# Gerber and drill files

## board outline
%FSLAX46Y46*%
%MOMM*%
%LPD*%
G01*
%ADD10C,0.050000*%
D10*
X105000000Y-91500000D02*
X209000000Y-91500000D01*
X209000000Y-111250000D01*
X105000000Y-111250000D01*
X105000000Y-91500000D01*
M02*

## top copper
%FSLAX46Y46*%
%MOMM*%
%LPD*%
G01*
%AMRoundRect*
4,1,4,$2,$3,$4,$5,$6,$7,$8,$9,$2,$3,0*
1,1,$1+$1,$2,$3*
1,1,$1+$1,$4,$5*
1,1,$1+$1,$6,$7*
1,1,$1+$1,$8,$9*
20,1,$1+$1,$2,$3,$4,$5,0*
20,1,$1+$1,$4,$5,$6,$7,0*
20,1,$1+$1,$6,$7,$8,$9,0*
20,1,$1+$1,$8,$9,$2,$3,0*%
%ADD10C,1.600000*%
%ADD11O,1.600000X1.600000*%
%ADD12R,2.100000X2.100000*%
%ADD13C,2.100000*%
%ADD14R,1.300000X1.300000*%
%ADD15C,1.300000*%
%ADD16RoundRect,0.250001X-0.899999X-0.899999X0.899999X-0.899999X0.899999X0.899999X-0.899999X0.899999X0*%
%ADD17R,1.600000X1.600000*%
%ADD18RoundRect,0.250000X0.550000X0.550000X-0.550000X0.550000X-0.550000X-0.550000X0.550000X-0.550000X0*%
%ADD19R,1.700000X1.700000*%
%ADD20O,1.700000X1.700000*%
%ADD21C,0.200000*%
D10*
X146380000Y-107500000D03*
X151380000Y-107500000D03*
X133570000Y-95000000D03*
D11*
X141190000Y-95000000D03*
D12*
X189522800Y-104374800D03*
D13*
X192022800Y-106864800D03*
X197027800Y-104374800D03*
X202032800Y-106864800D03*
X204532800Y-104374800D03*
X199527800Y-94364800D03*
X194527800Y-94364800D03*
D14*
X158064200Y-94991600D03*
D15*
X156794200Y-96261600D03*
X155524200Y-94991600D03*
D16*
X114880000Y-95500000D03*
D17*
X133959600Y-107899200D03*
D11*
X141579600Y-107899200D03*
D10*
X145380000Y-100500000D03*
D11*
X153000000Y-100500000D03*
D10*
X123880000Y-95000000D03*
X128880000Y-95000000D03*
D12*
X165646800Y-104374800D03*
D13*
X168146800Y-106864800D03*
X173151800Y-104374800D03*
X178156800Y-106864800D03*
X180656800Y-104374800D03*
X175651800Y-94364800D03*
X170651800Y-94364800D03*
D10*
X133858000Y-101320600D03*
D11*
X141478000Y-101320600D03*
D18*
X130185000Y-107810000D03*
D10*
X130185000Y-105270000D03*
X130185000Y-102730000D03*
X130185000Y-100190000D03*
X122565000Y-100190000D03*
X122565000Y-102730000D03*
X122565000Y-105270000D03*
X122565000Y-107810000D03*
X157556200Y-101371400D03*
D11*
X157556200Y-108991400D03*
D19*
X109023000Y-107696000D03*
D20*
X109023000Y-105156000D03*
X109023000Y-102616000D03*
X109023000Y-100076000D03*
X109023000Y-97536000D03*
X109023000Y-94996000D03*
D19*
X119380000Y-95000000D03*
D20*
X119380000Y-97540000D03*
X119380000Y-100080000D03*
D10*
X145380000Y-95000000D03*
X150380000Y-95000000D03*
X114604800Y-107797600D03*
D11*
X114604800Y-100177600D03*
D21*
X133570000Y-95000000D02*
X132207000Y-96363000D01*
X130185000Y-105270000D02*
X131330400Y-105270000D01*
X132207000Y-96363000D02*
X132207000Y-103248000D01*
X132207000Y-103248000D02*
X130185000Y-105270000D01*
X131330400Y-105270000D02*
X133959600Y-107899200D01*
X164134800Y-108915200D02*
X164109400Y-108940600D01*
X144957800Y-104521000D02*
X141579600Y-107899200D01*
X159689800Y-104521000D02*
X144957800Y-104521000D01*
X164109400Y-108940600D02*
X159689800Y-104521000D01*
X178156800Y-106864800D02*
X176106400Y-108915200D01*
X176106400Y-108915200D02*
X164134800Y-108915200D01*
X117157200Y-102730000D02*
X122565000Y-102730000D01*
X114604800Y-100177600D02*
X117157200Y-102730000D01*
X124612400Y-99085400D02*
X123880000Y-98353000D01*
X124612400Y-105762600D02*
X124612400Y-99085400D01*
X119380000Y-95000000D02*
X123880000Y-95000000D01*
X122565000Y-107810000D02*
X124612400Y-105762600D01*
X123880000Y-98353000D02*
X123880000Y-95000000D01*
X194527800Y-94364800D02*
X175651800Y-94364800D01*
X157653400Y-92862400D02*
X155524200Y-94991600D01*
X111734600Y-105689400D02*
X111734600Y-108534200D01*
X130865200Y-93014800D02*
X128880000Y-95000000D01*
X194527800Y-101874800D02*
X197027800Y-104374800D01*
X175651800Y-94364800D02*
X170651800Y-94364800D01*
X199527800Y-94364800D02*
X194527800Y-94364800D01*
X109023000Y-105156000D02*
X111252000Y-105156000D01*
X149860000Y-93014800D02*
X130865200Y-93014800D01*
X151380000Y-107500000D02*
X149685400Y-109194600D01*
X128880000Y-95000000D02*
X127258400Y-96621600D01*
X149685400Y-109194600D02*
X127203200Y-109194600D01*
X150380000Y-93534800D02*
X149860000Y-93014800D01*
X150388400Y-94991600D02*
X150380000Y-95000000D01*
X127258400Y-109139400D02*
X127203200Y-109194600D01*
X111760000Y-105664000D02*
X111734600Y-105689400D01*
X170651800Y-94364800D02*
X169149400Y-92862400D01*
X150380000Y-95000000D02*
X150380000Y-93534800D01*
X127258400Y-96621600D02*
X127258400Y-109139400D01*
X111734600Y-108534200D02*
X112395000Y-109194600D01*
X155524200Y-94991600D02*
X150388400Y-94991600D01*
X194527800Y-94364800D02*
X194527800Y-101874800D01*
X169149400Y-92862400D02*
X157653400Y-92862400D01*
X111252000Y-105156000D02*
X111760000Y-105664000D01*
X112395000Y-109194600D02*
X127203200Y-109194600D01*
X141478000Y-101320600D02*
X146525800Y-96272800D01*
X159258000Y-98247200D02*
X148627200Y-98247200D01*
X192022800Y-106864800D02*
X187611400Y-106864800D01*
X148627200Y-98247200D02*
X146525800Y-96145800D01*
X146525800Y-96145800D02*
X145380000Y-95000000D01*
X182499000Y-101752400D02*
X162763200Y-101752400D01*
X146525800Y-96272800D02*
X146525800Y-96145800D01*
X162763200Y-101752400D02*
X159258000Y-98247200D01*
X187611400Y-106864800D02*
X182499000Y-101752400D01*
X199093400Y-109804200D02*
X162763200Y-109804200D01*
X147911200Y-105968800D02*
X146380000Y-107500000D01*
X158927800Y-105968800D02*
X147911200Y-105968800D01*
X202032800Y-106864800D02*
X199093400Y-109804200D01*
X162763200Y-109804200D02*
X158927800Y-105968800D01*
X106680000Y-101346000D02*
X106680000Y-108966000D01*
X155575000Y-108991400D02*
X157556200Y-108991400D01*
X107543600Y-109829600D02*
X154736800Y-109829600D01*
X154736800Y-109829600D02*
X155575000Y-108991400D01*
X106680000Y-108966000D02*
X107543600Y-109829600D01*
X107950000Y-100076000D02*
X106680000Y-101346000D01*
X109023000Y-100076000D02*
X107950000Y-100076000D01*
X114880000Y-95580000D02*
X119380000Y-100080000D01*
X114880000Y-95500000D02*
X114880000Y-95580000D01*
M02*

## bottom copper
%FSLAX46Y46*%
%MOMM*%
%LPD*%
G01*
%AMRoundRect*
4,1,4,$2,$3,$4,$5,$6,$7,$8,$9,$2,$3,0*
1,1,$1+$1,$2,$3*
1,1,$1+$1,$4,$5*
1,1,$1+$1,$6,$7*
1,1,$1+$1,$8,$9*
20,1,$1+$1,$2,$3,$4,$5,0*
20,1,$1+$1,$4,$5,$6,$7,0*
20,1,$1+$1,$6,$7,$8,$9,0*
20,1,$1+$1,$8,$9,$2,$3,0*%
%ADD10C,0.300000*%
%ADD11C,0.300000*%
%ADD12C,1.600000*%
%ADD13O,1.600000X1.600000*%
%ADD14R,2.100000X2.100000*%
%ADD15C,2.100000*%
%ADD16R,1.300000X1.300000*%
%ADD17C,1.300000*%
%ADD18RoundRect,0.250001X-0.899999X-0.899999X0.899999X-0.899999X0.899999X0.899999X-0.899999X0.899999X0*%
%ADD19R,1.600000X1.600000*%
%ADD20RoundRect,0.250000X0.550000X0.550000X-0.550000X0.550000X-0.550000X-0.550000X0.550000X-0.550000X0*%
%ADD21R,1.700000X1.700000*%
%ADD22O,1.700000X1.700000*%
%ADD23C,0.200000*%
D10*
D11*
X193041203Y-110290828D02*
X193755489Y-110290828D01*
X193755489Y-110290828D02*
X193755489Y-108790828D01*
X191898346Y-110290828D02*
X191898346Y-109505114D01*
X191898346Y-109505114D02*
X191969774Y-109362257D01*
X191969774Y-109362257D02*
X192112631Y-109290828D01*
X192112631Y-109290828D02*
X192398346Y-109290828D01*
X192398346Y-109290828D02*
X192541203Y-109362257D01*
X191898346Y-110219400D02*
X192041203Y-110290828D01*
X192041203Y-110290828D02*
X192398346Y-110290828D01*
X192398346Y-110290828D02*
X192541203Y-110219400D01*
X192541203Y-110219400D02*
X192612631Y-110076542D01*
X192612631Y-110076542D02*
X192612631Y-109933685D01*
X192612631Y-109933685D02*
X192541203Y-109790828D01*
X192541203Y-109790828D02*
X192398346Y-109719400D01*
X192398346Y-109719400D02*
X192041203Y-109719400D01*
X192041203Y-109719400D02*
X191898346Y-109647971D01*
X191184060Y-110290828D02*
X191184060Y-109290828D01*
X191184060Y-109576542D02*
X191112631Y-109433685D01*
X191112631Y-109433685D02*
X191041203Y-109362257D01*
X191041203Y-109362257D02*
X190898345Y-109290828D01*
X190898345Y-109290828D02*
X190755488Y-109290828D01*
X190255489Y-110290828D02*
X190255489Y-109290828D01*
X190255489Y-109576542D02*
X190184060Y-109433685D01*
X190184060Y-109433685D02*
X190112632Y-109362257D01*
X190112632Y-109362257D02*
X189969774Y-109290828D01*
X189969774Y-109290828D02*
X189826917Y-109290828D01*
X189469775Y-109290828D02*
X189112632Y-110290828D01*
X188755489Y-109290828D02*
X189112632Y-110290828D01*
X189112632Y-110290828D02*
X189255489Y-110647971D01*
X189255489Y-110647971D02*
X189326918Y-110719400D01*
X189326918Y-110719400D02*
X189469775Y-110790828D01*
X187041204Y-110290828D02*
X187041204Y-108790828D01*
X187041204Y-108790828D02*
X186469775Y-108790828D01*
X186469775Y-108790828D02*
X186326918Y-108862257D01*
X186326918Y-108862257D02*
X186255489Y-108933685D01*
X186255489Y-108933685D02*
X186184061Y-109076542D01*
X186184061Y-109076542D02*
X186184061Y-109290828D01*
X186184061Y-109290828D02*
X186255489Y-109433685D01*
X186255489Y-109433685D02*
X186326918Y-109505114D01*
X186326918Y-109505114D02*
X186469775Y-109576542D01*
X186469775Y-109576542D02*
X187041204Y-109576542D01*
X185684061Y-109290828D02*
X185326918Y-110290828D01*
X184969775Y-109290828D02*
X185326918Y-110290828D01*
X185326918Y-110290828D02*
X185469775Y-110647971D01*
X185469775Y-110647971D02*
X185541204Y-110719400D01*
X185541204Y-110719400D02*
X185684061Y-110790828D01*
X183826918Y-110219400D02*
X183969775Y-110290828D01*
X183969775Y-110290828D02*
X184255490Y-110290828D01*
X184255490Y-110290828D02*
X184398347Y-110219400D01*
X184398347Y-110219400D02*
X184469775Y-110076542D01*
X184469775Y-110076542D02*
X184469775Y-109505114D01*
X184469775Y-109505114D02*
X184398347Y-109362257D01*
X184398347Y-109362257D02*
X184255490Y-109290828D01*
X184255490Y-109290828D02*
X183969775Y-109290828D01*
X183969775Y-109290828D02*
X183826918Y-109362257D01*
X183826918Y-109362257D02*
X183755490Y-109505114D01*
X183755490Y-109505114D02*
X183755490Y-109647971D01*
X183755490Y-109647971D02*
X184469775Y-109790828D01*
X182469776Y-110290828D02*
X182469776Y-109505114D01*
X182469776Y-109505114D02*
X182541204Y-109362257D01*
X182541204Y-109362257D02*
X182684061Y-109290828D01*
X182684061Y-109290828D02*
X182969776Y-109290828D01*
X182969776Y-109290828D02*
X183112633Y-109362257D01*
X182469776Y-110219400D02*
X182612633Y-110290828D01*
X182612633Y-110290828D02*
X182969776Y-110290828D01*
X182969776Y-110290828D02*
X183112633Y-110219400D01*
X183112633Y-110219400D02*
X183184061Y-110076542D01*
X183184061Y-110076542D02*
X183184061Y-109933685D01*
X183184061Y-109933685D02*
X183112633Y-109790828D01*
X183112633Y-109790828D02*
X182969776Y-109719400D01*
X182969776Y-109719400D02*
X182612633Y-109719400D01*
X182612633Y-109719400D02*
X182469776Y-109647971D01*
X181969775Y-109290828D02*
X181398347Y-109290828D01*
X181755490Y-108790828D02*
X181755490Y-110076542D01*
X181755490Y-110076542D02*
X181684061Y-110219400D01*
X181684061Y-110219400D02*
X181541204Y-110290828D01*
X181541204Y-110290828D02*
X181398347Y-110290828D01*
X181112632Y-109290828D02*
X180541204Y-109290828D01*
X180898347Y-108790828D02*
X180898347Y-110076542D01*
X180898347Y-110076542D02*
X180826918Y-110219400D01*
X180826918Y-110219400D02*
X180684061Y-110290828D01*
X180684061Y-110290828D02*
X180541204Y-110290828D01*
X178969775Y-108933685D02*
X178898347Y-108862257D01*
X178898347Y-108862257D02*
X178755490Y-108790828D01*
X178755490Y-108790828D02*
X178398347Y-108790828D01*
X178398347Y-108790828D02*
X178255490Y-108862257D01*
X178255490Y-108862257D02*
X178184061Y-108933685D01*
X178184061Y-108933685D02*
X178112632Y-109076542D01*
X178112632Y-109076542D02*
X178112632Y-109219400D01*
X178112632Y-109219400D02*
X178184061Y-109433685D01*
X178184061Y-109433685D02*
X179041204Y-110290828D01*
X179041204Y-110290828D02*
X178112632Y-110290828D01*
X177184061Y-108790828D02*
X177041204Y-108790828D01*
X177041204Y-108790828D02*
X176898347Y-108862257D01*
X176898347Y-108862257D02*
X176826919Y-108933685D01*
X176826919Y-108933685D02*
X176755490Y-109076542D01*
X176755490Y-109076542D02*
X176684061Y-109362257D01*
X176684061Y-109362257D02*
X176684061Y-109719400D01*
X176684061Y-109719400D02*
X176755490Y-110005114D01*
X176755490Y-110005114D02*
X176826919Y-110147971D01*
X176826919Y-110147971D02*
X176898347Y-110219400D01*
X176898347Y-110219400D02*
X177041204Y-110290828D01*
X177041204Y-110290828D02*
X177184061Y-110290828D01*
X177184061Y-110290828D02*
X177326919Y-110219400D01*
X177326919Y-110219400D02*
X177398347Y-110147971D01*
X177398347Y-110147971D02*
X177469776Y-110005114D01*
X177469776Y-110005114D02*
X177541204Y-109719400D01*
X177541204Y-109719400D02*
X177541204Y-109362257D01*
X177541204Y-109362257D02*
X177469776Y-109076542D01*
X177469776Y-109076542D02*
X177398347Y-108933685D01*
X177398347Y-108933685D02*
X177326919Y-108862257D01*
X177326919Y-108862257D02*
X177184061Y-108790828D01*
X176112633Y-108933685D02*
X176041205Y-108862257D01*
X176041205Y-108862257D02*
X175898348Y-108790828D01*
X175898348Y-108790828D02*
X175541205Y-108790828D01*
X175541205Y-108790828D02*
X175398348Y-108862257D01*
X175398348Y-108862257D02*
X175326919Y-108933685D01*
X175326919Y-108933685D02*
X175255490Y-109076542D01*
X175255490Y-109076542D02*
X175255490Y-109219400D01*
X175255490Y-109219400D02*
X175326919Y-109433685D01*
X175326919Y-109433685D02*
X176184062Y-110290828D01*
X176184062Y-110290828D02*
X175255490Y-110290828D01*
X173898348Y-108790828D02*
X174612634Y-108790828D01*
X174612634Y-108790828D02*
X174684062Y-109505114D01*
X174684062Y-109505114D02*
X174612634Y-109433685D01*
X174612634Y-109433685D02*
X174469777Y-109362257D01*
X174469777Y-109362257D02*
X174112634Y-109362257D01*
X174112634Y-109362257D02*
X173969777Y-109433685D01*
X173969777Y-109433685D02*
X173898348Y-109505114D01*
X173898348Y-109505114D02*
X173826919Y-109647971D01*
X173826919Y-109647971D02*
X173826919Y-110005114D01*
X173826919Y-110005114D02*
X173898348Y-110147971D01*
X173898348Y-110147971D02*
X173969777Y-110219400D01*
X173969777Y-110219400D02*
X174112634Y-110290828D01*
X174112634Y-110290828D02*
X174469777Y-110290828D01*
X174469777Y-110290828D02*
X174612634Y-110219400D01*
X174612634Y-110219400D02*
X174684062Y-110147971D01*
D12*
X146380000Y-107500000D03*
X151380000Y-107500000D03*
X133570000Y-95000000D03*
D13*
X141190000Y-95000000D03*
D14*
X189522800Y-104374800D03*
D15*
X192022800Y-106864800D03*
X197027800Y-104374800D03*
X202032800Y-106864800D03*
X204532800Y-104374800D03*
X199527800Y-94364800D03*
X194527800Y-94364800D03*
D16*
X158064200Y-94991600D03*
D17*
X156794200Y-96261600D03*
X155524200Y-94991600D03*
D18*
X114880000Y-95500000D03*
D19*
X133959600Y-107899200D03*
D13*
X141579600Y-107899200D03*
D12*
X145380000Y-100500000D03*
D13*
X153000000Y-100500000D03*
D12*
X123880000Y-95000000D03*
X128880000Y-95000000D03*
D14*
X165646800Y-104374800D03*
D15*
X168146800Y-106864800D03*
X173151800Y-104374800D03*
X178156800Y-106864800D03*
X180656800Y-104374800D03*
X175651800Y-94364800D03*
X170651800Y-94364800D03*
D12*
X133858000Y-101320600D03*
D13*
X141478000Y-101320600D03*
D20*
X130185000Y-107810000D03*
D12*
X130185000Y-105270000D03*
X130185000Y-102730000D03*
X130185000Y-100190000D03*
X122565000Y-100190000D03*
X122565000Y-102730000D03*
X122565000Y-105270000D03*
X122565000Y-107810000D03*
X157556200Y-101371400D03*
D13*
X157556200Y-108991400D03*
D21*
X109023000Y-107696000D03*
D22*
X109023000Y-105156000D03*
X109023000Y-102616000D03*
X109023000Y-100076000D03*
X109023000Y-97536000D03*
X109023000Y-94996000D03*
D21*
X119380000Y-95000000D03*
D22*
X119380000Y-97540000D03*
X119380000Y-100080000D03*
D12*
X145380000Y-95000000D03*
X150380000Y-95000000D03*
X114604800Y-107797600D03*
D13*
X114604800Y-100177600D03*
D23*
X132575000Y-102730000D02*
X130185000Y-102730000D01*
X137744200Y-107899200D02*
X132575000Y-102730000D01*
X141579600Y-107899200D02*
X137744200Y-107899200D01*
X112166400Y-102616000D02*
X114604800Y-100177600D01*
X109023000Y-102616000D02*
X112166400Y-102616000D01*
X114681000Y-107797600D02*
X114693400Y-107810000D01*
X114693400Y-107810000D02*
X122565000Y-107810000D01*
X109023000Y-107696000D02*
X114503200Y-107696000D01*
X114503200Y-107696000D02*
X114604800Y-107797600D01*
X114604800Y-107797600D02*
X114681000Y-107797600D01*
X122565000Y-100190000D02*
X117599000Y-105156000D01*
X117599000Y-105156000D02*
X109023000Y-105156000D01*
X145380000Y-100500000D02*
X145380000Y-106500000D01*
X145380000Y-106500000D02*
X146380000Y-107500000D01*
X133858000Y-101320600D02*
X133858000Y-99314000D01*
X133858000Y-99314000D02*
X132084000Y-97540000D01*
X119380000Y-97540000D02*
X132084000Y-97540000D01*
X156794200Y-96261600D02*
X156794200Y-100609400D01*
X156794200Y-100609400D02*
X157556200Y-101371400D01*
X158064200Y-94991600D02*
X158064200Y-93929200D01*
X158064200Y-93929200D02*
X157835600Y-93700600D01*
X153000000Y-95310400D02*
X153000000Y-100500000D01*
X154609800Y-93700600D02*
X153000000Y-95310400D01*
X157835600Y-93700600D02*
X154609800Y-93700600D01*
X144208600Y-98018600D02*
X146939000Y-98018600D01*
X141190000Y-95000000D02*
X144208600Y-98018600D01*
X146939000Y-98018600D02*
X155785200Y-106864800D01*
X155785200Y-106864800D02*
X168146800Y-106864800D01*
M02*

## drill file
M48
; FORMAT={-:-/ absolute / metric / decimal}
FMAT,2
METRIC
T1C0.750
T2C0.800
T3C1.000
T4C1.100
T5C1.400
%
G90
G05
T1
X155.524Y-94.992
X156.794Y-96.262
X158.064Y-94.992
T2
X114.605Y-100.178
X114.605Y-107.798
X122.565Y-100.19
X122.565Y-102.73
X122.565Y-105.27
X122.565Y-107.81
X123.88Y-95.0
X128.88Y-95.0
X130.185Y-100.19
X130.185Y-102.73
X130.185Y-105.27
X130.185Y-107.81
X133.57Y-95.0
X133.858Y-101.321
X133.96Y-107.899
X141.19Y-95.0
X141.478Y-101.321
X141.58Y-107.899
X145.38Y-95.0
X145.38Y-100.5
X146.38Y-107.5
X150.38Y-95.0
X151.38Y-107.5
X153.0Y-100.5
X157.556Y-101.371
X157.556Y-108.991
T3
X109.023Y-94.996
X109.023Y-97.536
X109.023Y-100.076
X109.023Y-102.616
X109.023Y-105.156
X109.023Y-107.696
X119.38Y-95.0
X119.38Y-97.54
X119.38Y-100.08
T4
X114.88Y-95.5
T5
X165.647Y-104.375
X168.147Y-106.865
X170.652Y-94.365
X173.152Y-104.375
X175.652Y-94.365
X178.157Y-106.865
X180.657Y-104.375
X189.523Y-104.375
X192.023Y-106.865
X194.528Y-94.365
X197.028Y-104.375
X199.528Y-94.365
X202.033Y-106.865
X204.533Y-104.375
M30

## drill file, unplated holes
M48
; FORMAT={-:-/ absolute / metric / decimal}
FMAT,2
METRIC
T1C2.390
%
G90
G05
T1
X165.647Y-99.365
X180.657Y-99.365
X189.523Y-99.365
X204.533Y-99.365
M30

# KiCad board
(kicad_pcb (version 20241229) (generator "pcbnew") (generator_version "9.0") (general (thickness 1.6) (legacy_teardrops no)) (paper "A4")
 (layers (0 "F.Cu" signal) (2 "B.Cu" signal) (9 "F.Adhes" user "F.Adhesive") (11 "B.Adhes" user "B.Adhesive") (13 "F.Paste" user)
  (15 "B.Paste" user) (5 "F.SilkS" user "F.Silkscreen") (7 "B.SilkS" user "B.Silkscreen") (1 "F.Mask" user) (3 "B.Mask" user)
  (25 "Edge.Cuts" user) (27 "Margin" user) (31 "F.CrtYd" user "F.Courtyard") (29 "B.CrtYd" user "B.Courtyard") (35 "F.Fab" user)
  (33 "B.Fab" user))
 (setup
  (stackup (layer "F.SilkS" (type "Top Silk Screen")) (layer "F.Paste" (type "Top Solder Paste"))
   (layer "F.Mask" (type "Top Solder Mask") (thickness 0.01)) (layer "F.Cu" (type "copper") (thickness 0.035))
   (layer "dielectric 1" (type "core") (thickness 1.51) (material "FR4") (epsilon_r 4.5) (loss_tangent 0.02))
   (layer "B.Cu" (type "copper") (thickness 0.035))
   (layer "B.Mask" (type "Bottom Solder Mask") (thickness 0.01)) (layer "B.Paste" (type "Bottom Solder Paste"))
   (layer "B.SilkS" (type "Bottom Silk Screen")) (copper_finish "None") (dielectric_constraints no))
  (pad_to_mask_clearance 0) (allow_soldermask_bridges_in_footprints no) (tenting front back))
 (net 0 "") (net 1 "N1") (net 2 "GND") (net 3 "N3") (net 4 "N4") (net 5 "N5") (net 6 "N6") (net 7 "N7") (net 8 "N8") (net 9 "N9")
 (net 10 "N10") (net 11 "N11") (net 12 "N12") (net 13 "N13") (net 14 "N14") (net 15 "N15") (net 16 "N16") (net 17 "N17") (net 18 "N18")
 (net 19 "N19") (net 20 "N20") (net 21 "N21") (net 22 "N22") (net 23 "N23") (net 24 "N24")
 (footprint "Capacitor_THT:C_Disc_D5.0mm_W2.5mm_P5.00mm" (layer "F.Cu") (at 146.38 107.5)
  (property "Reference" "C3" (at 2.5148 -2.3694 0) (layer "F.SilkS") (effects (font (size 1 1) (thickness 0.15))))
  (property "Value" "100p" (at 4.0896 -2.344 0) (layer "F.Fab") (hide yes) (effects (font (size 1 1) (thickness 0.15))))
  (pad "1" thru_hole circle (at 0 0) (size 1.6 1.6) (drill 0.8) (layers "*.Cu" "*.Mask") (remove_unused_layers no) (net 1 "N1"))
  (pad "2" thru_hole circle (at 5 0) (size 1.6 1.6) (drill 0.8) (layers "*.Cu" "*.Mask") (remove_unused_layers no) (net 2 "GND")))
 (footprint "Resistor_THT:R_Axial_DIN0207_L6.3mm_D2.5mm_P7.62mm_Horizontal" (layer "F.Cu") (at 133.57 95)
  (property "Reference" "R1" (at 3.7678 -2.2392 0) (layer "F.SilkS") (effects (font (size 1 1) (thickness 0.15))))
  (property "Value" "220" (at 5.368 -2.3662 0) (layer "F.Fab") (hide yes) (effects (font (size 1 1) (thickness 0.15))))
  (pad "1" thru_hole circle (at 0 0) (size 1.6 1.6) (drill 0.8) (layers "*.Cu" "*.Mask") (remove_unused_layers no) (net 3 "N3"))
  (pad "2" thru_hole oval (at 7.62 0) (size 1.6 1.6) (drill 0.8) (layers "*.Cu" "*.Mask") (remove_unused_layers no) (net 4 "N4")))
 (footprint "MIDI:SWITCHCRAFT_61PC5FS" (layer "F.Cu") (at 197.0278 99.3648 -90)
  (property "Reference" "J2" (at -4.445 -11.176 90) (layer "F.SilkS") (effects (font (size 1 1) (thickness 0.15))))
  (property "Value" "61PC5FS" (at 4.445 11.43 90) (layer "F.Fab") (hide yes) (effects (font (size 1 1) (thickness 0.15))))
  (pad "" np_thru_hole circle (at 0 -7.505 270) (size 2.39 2.39) (drill 2.39) (layers "*.Cu" "*.Mask"))
  (pad "" np_thru_hole circle (at 0 7.505 270) (size 2.39 2.39) (drill 2.39) (layers "*.Cu" "*.Mask"))
  (pad "1" thru_hole rect (at 5.01 7.505 270) (size 2.1 2.1) (drill 1.4) (layers "*.Cu" "*.Mask") (remove_unused_layers no) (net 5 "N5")
   (solder_mask_margin 0.102))
  (pad "2" thru_hole circle (at 7.5 5.005 270) (size 2.1 2.1) (drill 1.4) (layers "*.Cu" "*.Mask") (remove_unused_layers no) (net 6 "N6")
   (solder_mask_margin 0.102))
  (pad "3" thru_hole circle (at 5.01 0 270) (size 2.1 2.1) (drill 1.4) (layers "*.Cu" "*.Mask") (remove_unused_layers no) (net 2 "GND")
   (solder_mask_margin 0.102))
  (pad "4" thru_hole circle (at 7.5 -5.005 270) (size 2.1 2.1) (drill 1.4) (layers "*.Cu" "*.Mask") (remove_unused_layers no) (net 1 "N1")
   (solder_mask_margin 0.102))
  (pad "5" thru_hole circle (at 5.01 -7.505 270) (size 2.1 2.1) (drill 1.4) (layers "*.Cu" "*.Mask") (remove_unused_layers no) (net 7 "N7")
   (solder_mask_margin 0.102))
  (pad "G1" thru_hole circle (at -5 -2.5 270) (size 2.1 2.1) (drill 1.4) (layers "*.Cu" "*.Mask") (remove_unused_layers no) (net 2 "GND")
   (solder_mask_margin 0.102))
  (pad "G2" thru_hole circle (at -5 2.5 270) (size 2.1 2.1) (drill 1.4) (layers "*.Cu" "*.Mask") (remove_unused_layers no) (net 2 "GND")
   (solder_mask_margin 0.102)))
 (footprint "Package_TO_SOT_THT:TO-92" (layer "F.Cu") (at 158.0642 94.9916 180)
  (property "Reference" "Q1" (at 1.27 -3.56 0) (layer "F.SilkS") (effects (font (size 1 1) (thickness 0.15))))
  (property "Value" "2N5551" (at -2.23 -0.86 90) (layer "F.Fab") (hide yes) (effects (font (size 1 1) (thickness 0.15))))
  (pad "1" thru_hole rect (at 0 0 180) (size 1.3 1.3) (drill 0.75) (layers "*.Cu" "*.Mask") (remove_unused_layers no) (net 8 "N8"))
  (pad "2" thru_hole circle (at 1.27 -1.27 180) (size 1.3 1.3) (drill 0.75) (layers "*.Cu" "*.Mask") (remove_unused_layers no) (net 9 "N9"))
  (pad "3" thru_hole circle (at 2.54 0 180) (size 1.3 1.3) (drill 0.75) (layers "*.Cu" "*.Mask") (remove_unused_layers no) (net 2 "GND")))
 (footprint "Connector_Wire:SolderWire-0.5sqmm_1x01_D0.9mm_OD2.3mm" (layer "F.Cu") (at 114.88 95.5)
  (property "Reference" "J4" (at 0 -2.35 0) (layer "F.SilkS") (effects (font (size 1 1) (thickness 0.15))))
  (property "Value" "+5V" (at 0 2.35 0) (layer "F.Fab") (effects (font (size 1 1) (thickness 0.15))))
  (pad "1" thru_hole roundrect (at 0 0) (size 2.3 2.3) (drill 1.1) (layers "*.Cu" "*.Mask") (remove_unused_layers no)
   (roundrect_rratio 0.108696) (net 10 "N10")))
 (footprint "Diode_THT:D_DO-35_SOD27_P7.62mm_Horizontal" (layer "F.Cu") (at 133.9596 107.8992)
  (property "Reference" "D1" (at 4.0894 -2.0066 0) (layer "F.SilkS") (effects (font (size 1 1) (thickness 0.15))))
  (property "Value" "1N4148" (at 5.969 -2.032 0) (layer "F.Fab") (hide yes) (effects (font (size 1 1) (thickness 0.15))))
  (pad "1" thru_hole rect (at 0 0) (size 1.6 1.6) (drill 0.8) (layers "*.Cu" "*.Mask") (remove_unused_layers no) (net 3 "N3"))
  (pad "2" thru_hole oval (at 7.62 0) (size 1.6 1.6) (drill 0.8) (layers "*.Cu" "*.Mask") (remove_unused_layers no) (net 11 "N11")))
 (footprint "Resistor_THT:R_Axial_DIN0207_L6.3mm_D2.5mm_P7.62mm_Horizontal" (layer "F.Cu") (at 145.38 100.5)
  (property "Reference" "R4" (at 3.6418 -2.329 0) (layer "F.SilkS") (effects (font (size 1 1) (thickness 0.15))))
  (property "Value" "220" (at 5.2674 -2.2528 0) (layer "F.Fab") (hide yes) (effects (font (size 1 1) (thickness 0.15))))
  (pad "1" thru_hole circle (at 0 0) (size 1.6 1.6) (drill 0.8) (layers "*.Cu" "*.Mask") (remove_unused_layers no) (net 1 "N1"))
  (pad "2" thru_hole oval (at 7.62 0) (size 1.6 1.6) (drill 0.8) (layers "*.Cu" "*.Mask") (remove_unused_layers no) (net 8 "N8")))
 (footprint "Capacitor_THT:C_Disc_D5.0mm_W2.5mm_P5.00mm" (layer "F.Cu") (at 123.88 95)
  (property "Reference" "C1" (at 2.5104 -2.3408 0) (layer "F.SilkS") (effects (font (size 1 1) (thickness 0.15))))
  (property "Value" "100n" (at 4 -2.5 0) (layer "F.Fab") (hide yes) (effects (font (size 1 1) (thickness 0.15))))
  (pad "1" thru_hole circle (at 0 0) (size 1.6 1.6) (drill 0.8) (layers "*.Cu" "*.Mask") (remove_unused_layers no) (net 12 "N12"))
  (pad "2" thru_hole circle (at 5 0) (size 1.6 1.6) (drill 0.8) (layers "*.Cu" "*.Mask") (remove_unused_layers no) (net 2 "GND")))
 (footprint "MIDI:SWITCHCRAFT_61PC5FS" (layer "F.Cu") (at 173.1518 99.3648 -90)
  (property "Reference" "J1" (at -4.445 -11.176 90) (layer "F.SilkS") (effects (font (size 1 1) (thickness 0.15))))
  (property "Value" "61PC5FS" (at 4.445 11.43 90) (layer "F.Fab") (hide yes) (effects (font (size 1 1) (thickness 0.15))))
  (pad "" np_thru_hole circle (at 0 -7.505 270) (size 2.39 2.39) (drill 2.39) (layers "*.Cu" "*.Mask"))
  (pad "" np_thru_hole circle (at 0 7.505 270) (size 2.39 2.39) (drill 2.39) (layers "*.Cu" "*.Mask"))
  (pad "1" thru_hole rect (at 5.01 7.505 270) (size 2.1 2.1) (drill 1.4) (layers "*.Cu" "*.Mask") (remove_unused_layers no) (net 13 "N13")
   (solder_mask_margin 0.102))
  (pad "2" thru_hole circle (at 7.5 5.005 270) (size 2.1 2.1) (drill 1.4) (layers "*.Cu" "*.Mask") (remove_unused_layers no) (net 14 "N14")
   (solder_mask_margin 0.102))
  (pad "3" thru_hole circle (at 5.01 0 270) (size 2.1 2.1) (drill 1.4) (layers "*.Cu" "*.Mask") (remove_unused_layers no) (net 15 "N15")
   (solder_mask_margin 0.102))
  (pad "4" thru_hole circle (at 7.5 -5.005 270) (size 2.1 2.1) (drill 1.4) (layers "*.Cu" "*.Mask") (remove_unused_layers no) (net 11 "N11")
   (solder_mask_margin 0.102))
  (pad "5" thru_hole circle (at 5.01 -7.505 270) (size 2.1 2.1) (drill 1.4) (layers "*.Cu" "*.Mask") (remove_unused_layers no)
   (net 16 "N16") (solder_mask_margin 0.102))
  (pad "G1" thru_hole circle (at -5 -2.5 270) (size 2.1 2.1) (drill 1.4) (layers "*.Cu" "*.Mask") (remove_unused_layers no) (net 2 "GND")
   (solder_mask_margin 0.102))
  (pad "G2" thru_hole circle (at -5 2.5 270) (size 2.1 2.1) (drill 1.4) (layers "*.Cu" "*.Mask") (remove_unused_layers no) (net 2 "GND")
   (solder_mask_margin 0.102)))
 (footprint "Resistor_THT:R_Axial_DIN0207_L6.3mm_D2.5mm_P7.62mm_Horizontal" (layer "F.Cu") (at 133.858 101.3206)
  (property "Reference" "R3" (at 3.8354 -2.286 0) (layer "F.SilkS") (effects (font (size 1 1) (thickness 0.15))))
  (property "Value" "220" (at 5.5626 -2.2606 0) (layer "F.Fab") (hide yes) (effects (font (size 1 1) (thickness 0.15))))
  (pad "1" thru_hole circle (at 0 0) (size 1.6 1.6) (drill 0.8) (layers "*.Cu" "*.Mask") (remove_unused_layers no) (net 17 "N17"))
  (pad "2" thru_hole oval (at 7.62 0) (size 1.6 1.6) (drill 0.8) (layers "*.Cu" "*.Mask") (remove_unused_layers no) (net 6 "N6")))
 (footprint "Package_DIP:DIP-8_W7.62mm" (layer "F.Cu") (at 130.185 107.81 180)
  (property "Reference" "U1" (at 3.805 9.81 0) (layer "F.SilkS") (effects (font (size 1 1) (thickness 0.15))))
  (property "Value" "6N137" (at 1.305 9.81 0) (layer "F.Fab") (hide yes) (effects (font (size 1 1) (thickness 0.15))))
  (pad "1" thru_hole roundrect (at 0 0 180) (size 1.6 1.6) (drill 0.8) (layers "*.Cu" "*.Mask") (remove_unused_layers no)
   (roundrect_rratio 0.15625) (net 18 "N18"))
  (pad "2" thru_hole circle (at 0 2.54 180) (size 1.6 1.6) (drill 0.8) (layers "*.Cu" "*.Mask") (remove_unused_layers no) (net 3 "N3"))
  (pad "3" thru_hole circle (at 0 5.08 180) (size 1.6 1.6) (drill 0.8) (layers "*.Cu" "*.Mask") (remove_unused_layers no) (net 11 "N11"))
  (pad "4" thru_hole circle (at 0 7.62 180) (size 1.6 1.6) (drill 0.8) (layers "*.Cu" "*.Mask") (remove_unused_layers no) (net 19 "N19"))
  (pad "5" thru_hole circle (at 7.62 7.62 180) (size 1.6 1.6) (drill 0.8) (layers "*.Cu" "*.Mask") (remove_unused_layers no) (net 2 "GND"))
  (pad "6" thru_hole circle (at 7.62 5.08 180) (size 1.6 1.6) (drill 0.8) (layers "*.Cu" "*.Mask") (remove_unused_layers no) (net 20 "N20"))
  (pad "7" thru_hole circle (at 7.62 2.54 180) (size 1.6 1.6) (drill 0.8) (layers "*.Cu" "*.Mask") (remove_unused_layers no) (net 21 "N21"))
  (pad "8" thru_hole circle (at 7.62 0 180) (size 1.6 1.6) (drill 0.8) (layers "*.Cu" "*.Mask") (remove_unused_layers no) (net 12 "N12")))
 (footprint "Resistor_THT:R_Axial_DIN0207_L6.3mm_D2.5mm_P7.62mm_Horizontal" (layer "F.Cu") (at 157.5562 101.3714 -90)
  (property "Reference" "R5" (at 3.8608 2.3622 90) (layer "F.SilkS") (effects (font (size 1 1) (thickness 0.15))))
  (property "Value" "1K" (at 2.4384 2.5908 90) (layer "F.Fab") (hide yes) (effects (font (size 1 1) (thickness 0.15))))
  (pad "1" thru_hole circle (at 0 0 270) (size 1.6 1.6) (drill 0.8) (layers "*.Cu" "*.Mask") (remove_unused_layers no) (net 9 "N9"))
  (pad "2" thru_hole oval (at 7.62 0 270) (size 1.6 1.6) (drill 0.8) (layers "*.Cu" "*.Mask") (remove_unused_layers no) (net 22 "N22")))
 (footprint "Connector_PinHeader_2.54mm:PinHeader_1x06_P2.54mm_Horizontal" (layer "F.Cu") (at 109.023 107.696 180)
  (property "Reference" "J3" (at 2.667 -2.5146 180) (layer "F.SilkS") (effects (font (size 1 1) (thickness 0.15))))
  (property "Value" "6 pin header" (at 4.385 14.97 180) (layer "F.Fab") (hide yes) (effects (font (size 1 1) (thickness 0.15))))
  (pad "1" thru_hole rect (at 0 0 180) (size 1.7 1.7) (drill 1) (layers "*.Cu" "*.Mask") (remove_unused_layers no) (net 12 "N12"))
  (pad "2" thru_hole oval (at 0 2.54 180) (size 1.7 1.7) (drill 1) (layers "*.Cu" "*.Mask") (remove_unused_layers no) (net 2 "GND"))
  (pad "3" thru_hole oval (at 0 5.08 180) (size 1.7 1.7) (drill 1) (layers "*.Cu" "*.Mask") (remove_unused_layers no) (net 20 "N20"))
  (pad "4" thru_hole oval (at 0 7.62 180) (size 1.7 1.7) (drill 1) (layers "*.Cu" "*.Mask") (remove_unused_layers no) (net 22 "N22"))
  (pad "5" thru_hole oval (at 0 10.16 180) (size 1.7 1.7) (drill 1) (layers "*.Cu" "*.Mask") (remove_unused_layers no) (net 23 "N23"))
  (pad "6" thru_hole oval (at 0 12.7 180) (size 1.7 1.7) (drill 1) (layers "*.Cu" "*.Mask") (remove_unused_layers no) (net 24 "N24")))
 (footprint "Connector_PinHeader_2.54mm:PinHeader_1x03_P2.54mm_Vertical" (layer "F.Cu") (at 119.38 95)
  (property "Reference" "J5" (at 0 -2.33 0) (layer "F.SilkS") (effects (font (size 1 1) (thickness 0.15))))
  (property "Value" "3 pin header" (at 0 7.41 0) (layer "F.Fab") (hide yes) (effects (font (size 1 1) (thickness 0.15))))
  (pad "1" thru_hole rect (at 0 0) (size 1.7 1.7) (drill 1) (layers "*.Cu" "*.Mask") (remove_unused_layers no) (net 12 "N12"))
  (pad "2" thru_hole oval (at 0 2.54) (size 1.7 1.7) (drill 1) (layers "*.Cu" "*.Mask") (remove_unused_layers no) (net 17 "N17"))
  (pad "3" thru_hole oval (at 0 5.08) (size 1.7 1.7) (drill 1) (layers "*.Cu" "*.Mask") (remove_unused_layers no) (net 10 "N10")))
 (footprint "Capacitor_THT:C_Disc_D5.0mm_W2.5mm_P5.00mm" (layer "F.Cu") (at 145.38 95)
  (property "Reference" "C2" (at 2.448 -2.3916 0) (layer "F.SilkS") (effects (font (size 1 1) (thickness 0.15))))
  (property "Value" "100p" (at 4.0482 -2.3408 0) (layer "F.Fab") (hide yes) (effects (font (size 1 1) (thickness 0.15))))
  (pad "1" thru_hole circle (at 0 0) (size 1.6 1.6) (drill 0.8) (layers "*.Cu" "*.Mask") (remove_unused_layers no) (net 6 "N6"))
  (pad "2" thru_hole circle (at 5 0) (size 1.6 1.6) (drill 0.8) (layers "*.Cu" "*.Mask") (remove_unused_layers no) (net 2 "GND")))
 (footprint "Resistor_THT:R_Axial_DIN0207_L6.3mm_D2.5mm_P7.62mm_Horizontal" (layer "F.Cu") (at 114.6048 107.7976 90)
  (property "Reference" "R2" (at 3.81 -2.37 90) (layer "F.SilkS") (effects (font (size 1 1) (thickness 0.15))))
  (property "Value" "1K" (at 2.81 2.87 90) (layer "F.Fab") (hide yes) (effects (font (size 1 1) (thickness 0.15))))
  (pad "1" thru_hole circle (at 0 0 90) (size 1.6 1.6) (drill 0.8) (layers "*.Cu" "*.Mask") (remove_unused_layers no) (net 12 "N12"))
  (pad "2" thru_hole oval (at 7.62 0 90) (size 1.6 1.6) (drill 0.8) (layers "*.Cu" "*.Mask") (remove_unused_layers no) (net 20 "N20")))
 (gr_rect (start 105 91.5) (end 209 111.25) (stroke (width 0.05) (type solid)) (fill no) (layer "Edge.Cuts"))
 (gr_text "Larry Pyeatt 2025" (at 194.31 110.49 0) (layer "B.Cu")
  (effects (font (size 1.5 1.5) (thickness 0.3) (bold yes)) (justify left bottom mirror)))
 (segment (start 133.57 95) (end 132.207 96.363) (width 0.2) (layer "F.Cu") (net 3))
 (segment (start 130.185 105.27) (end 131.3304 105.27) (width 0.2) (layer "F.Cu") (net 3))
 (segment (start 132.207 96.363) (end 132.207 103.248) (width 0.2) (layer "F.Cu") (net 3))
 (segment (start 132.207 103.248) (end 130.185 105.27) (width 0.2) (layer "F.Cu") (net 3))
 (segment (start 131.3304 105.27) (end 133.9596 107.8992) (width 0.2) (layer "F.Cu") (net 3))
 (segment (start 164.1348 108.9152) (end 164.1094 108.9406) (width 0.2) (layer "F.Cu") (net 11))
 (segment (start 144.9578 104.521) (end 141.5796 107.8992) (width 0.2) (layer "F.Cu") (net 11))
 (segment (start 159.6898 104.521) (end 144.9578 104.521) (width 0.2) (layer "F.Cu") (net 11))
 (segment (start 164.1094 108.9406) (end 159.6898 104.521) (width 0.2) (layer "F.Cu") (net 11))
 (segment (start 178.1568 106.8648) (end 176.1064 108.9152) (width 0.2) (layer "F.Cu") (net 11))
 (segment (start 176.1064 108.9152) (end 164.1348 108.9152) (width 0.2) (layer "F.Cu") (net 11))
 (segment (start 132.575 102.73) (end 130.185 102.73) (width 0.2) (layer "B.Cu") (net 11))
 (segment (start 137.7442 107.8992) (end 132.575 102.73) (width 0.2) (layer "B.Cu") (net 11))
 (segment (start 141.5796 107.8992) (end 137.7442 107.8992) (width 0.2) (layer "B.Cu") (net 11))
 (segment (start 117.1572 102.73) (end 122.565 102.73) (width 0.2) (layer "F.Cu") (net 20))
 (segment (start 114.6048 100.1776) (end 117.1572 102.73) (width 0.2) (layer "F.Cu") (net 20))
 (segment (start 112.1664 102.616) (end 114.6048 100.1776) (width 0.2) (layer "B.Cu") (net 20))
 (segment (start 109.023 102.616) (end 112.1664 102.616) (width 0.2) (layer "B.Cu") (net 20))
 (segment (start 124.6124 99.0854) (end 123.88 98.353) (width 0.2) (layer "F.Cu") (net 12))
 (segment (start 124.6124 105.7626) (end 124.6124 99.0854) (width 0.2) (layer "F.Cu") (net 12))
 (segment (start 119.38 95) (end 123.88 95) (width 0.2) (layer "F.Cu") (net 12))
 (segment (start 122.565 107.81) (end 124.6124 105.7626) (width 0.2) (layer "F.Cu") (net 12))
 (segment (start 123.88 98.353) (end 123.88 95) (width 0.2) (layer "F.Cu") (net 12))
 (segment (start 114.681 107.7976) (end 114.6934 107.81) (width 0.2) (layer "B.Cu") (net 12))
 (segment (start 114.6934 107.81) (end 122.565 107.81) (width 0.2) (layer "B.Cu") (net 12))
 (segment (start 109.023 107.696) (end 114.5032 107.696) (width 0.2) (layer "B.Cu") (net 12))
 (segment (start 114.5032 107.696) (end 114.6048 107.7976) (width 0.2) (layer "B.Cu") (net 12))
 (segment (start 114.6048 107.7976) (end 114.681 107.7976) (width 0.2) (layer "B.Cu") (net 12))
 (segment (start 194.5278 94.3648) (end 175.6518 94.3648) (width 0.2) (layer "F.Cu") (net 2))
 (segment (start 157.6534 92.8624) (end 155.5242 94.9916) (width 0.2) (layer "F.Cu") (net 2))
 (segment (start 111.7346 105.6894) (end 111.7346 108.5342) (width 0.2) (layer "F.Cu") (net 2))
 (segment (start 130.8652 93.0148) (end 128.88 95) (width 0.2) (layer "F.Cu") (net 2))
 (segment (start 194.5278 101.8748) (end 197.0278 104.3748) (width 0.2) (layer "F.Cu") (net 2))
 (segment (start 175.6518 94.3648) (end 170.6518 94.3648) (width 0.2) (layer "F.Cu") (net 2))
 (segment (start 199.5278 94.3648) (end 194.5278 94.3648) (width 0.2) (layer "F.Cu") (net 2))
 (segment (start 109.023 105.156) (end 111.252 105.156) (width 0.2) (layer "F.Cu") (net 2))
 (segment (start 149.86 93.0148) (end 130.8652 93.0148) (width 0.2) (layer "F.Cu") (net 2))
 (segment (start 151.38 107.5) (end 149.6854 109.1946) (width 0.2) (layer "F.Cu") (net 2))
 (segment (start 128.88 95) (end 127.2584 96.6216) (width 0.2) (layer "F.Cu") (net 2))
 (segment (start 149.6854 109.1946) (end 127.2032 109.1946) (width 0.2) (layer "F.Cu") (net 2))
 (segment (start 150.38 93.5348) (end 149.86 93.0148) (width 0.2) (layer "F.Cu") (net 2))
 (segment (start 150.3884 94.9916) (end 150.38 95) (width 0.2) (layer "F.Cu") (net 2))
 (segment (start 127.2584 109.1394) (end 127.2032 109.1946) (width 0.2) (layer "F.Cu") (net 2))
 (segment (start 111.76 105.664) (end 111.7346 105.6894) (width 0.2) (layer "F.Cu") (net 2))
 (segment (start 170.6518 94.3648) (end 169.1494 92.8624) (width 0.2) (layer "F.Cu") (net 2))
 (segment (start 150.38 95) (end 150.38 93.5348) (width 0.2) (layer "F.Cu") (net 2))
 (segment (start 127.2584 96.6216) (end 127.2584 109.1394) (width 0.2) (layer "F.Cu") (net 2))
 (segment (start 111.7346 108.5342) (end 112.395 109.1946) (width 0.2) (layer "F.Cu") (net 2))
 (segment (start 155.5242 94.9916) (end 150.3884 94.9916) (width 0.2) (layer "F.Cu") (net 2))
 (segment (start 194.5278 94.3648) (end 194.5278 101.8748) (width 0.2) (layer "F.Cu") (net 2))
 (segment (start 169.1494 92.8624) (end 157.6534 92.8624) (width 0.2) (layer "F.Cu") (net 2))
 (segment (start 111.252 105.156) (end 111.76 105.664) (width 0.2) (layer "F.Cu") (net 2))
 (segment (start 112.395 109.1946) (end 127.2032 109.1946) (width 0.2) (layer "F.Cu") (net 2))
 (segment (start 122.565 100.19) (end 117.599 105.156) (width 0.2) (layer "B.Cu") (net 2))
 (segment (start 117.599 105.156) (end 109.023 105.156) (width 0.2) (layer "B.Cu") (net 2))
 (segment (start 141.478 101.3206) (end 146.5258 96.2728) (width 0.2) (layer "F.Cu") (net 6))
 (segment (start 159.258 98.2472) (end 148.6272 98.2472) (width 0.2) (layer "F.Cu") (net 6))
 (segment (start 192.0228 106.8648) (end 187.6114 106.8648) (width 0.2) (layer "F.Cu") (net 6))
 (segment (start 148.6272 98.2472) (end 146.5258 96.1458) (width 0.2) (layer "F.Cu") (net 6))
 (segment (start 146.5258 96.1458) (end 145.38 95) (width 0.2) (layer "F.Cu") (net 6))
 (segment (start 182.499 101.7524) (end 162.7632 101.7524) (width 0.2) (layer "F.Cu") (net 6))
 (segment (start 146.5258 96.2728) (end 146.5258 96.1458) (width 0.2) (layer "F.Cu") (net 6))
 (segment (start 162.7632 101.7524) (end 159.258 98.2472) (width 0.2) (layer "F.Cu") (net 6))
 (segment (start 187.6114 106.8648) (end 182.499 101.7524) (width 0.2) (layer "F.Cu") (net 6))
 (segment (start 199.0934 109.8042) (end 162.7632 109.8042) (width 0.2) (layer "F.Cu") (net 1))
 (segment (start 147.9112 105.9688) (end 146.38 107.5) (width 0.2) (layer "F.Cu") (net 1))
 (segment (start 158.9278 105.9688) (end 147.9112 105.9688) (width 0.2) (layer "F.Cu") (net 1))
 (segment (start 202.0328 106.8648) (end 199.0934 109.8042) (width 0.2) (layer "F.Cu") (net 1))
 (segment (start 162.7632 109.8042) (end 158.9278 105.9688) (width 0.2) (layer "F.Cu") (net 1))
 (segment (start 145.38 100.5) (end 145.38 106.5) (width 0.2) (layer "B.Cu") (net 1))
 (segment (start 145.38 106.5) (end 146.38 107.5) (width 0.2) (layer "B.Cu") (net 1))
 (segment (start 106.68 101.346) (end 106.68 108.966) (width 0.2) (layer "F.Cu") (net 22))
 (segment (start 155.575 108.9914) (end 157.5562 108.9914) (width 0.2) (layer "F.Cu") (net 22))
 (segment (start 107.5436 109.8296) (end 154.7368 109.8296) (width 0.2) (layer "F.Cu") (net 22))
 (segment (start 154.7368 109.8296) (end 155.575 108.9914) (width 0.2) (layer "F.Cu") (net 22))
 (segment (start 106.68 108.966) (end 107.5436 109.8296) (width 0.2) (layer "F.Cu") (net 22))
 (segment (start 107.95 100.076) (end 106.68 101.346) (width 0.2) (layer "F.Cu") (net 22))
 (segment (start 109.023 100.076) (end 107.95 100.076) (width 0.2) (layer "F.Cu") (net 22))
 (segment (start 114.88 95.58) (end 119.38 100.08) (width 0.2) (layer "F.Cu") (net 10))
 (segment (start 114.88 95.5) (end 114.88 95.58) (width 0.2) (layer "F.Cu") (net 10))
 (segment (start 133.858 101.3206) (end 133.858 99.314) (width 0.2) (layer "B.Cu") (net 17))
 (segment (start 133.858 99.314) (end 132.084 97.54) (width 0.2) (layer "B.Cu") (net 17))
 (segment (start 119.38 97.54) (end 132.084 97.54) (width 0.2) (layer "B.Cu") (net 17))
 (segment (start 156.7942 96.2616) (end 156.7942 100.6094) (width 0.2) (layer "B.Cu") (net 9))
 (segment (start 156.7942 100.6094) (end 157.5562 101.3714) (width 0.2) (layer "B.Cu") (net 9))
 (segment (start 158.0642 94.9916) (end 158.0642 93.9292) (width 0.2) (layer "B.Cu") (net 8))
 (segment (start 158.0642 93.9292) (end 157.8356 93.7006) (width 0.2) (layer "B.Cu") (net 8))
 (segment (start 153 95.3104) (end 153 100.5) (width 0.2) (layer "B.Cu") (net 8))
 (segment (start 154.6098 93.7006) (end 153 95.3104) (width 0.2) (layer "B.Cu") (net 8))
 (segment (start 157.8356 93.7006) (end 154.6098 93.7006) (width 0.2) (layer "B.Cu") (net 8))
 (segment (start 144.2086 98.0186) (end 146.939 98.0186) (width 0.2) (layer "B.Cu") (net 14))
 (segment (start 141.19 95) (end 144.2086 98.0186) (width 0.2) (layer "B.Cu") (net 14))
 (segment (start 146.939 98.0186) (end 155.7852 106.8648) (width 0.2) (layer "B.Cu") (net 14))
 (segment (start 155.7852 106.8648) (end 168.1468 106.8648) (width 0.2) (layer "B.Cu") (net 14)))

